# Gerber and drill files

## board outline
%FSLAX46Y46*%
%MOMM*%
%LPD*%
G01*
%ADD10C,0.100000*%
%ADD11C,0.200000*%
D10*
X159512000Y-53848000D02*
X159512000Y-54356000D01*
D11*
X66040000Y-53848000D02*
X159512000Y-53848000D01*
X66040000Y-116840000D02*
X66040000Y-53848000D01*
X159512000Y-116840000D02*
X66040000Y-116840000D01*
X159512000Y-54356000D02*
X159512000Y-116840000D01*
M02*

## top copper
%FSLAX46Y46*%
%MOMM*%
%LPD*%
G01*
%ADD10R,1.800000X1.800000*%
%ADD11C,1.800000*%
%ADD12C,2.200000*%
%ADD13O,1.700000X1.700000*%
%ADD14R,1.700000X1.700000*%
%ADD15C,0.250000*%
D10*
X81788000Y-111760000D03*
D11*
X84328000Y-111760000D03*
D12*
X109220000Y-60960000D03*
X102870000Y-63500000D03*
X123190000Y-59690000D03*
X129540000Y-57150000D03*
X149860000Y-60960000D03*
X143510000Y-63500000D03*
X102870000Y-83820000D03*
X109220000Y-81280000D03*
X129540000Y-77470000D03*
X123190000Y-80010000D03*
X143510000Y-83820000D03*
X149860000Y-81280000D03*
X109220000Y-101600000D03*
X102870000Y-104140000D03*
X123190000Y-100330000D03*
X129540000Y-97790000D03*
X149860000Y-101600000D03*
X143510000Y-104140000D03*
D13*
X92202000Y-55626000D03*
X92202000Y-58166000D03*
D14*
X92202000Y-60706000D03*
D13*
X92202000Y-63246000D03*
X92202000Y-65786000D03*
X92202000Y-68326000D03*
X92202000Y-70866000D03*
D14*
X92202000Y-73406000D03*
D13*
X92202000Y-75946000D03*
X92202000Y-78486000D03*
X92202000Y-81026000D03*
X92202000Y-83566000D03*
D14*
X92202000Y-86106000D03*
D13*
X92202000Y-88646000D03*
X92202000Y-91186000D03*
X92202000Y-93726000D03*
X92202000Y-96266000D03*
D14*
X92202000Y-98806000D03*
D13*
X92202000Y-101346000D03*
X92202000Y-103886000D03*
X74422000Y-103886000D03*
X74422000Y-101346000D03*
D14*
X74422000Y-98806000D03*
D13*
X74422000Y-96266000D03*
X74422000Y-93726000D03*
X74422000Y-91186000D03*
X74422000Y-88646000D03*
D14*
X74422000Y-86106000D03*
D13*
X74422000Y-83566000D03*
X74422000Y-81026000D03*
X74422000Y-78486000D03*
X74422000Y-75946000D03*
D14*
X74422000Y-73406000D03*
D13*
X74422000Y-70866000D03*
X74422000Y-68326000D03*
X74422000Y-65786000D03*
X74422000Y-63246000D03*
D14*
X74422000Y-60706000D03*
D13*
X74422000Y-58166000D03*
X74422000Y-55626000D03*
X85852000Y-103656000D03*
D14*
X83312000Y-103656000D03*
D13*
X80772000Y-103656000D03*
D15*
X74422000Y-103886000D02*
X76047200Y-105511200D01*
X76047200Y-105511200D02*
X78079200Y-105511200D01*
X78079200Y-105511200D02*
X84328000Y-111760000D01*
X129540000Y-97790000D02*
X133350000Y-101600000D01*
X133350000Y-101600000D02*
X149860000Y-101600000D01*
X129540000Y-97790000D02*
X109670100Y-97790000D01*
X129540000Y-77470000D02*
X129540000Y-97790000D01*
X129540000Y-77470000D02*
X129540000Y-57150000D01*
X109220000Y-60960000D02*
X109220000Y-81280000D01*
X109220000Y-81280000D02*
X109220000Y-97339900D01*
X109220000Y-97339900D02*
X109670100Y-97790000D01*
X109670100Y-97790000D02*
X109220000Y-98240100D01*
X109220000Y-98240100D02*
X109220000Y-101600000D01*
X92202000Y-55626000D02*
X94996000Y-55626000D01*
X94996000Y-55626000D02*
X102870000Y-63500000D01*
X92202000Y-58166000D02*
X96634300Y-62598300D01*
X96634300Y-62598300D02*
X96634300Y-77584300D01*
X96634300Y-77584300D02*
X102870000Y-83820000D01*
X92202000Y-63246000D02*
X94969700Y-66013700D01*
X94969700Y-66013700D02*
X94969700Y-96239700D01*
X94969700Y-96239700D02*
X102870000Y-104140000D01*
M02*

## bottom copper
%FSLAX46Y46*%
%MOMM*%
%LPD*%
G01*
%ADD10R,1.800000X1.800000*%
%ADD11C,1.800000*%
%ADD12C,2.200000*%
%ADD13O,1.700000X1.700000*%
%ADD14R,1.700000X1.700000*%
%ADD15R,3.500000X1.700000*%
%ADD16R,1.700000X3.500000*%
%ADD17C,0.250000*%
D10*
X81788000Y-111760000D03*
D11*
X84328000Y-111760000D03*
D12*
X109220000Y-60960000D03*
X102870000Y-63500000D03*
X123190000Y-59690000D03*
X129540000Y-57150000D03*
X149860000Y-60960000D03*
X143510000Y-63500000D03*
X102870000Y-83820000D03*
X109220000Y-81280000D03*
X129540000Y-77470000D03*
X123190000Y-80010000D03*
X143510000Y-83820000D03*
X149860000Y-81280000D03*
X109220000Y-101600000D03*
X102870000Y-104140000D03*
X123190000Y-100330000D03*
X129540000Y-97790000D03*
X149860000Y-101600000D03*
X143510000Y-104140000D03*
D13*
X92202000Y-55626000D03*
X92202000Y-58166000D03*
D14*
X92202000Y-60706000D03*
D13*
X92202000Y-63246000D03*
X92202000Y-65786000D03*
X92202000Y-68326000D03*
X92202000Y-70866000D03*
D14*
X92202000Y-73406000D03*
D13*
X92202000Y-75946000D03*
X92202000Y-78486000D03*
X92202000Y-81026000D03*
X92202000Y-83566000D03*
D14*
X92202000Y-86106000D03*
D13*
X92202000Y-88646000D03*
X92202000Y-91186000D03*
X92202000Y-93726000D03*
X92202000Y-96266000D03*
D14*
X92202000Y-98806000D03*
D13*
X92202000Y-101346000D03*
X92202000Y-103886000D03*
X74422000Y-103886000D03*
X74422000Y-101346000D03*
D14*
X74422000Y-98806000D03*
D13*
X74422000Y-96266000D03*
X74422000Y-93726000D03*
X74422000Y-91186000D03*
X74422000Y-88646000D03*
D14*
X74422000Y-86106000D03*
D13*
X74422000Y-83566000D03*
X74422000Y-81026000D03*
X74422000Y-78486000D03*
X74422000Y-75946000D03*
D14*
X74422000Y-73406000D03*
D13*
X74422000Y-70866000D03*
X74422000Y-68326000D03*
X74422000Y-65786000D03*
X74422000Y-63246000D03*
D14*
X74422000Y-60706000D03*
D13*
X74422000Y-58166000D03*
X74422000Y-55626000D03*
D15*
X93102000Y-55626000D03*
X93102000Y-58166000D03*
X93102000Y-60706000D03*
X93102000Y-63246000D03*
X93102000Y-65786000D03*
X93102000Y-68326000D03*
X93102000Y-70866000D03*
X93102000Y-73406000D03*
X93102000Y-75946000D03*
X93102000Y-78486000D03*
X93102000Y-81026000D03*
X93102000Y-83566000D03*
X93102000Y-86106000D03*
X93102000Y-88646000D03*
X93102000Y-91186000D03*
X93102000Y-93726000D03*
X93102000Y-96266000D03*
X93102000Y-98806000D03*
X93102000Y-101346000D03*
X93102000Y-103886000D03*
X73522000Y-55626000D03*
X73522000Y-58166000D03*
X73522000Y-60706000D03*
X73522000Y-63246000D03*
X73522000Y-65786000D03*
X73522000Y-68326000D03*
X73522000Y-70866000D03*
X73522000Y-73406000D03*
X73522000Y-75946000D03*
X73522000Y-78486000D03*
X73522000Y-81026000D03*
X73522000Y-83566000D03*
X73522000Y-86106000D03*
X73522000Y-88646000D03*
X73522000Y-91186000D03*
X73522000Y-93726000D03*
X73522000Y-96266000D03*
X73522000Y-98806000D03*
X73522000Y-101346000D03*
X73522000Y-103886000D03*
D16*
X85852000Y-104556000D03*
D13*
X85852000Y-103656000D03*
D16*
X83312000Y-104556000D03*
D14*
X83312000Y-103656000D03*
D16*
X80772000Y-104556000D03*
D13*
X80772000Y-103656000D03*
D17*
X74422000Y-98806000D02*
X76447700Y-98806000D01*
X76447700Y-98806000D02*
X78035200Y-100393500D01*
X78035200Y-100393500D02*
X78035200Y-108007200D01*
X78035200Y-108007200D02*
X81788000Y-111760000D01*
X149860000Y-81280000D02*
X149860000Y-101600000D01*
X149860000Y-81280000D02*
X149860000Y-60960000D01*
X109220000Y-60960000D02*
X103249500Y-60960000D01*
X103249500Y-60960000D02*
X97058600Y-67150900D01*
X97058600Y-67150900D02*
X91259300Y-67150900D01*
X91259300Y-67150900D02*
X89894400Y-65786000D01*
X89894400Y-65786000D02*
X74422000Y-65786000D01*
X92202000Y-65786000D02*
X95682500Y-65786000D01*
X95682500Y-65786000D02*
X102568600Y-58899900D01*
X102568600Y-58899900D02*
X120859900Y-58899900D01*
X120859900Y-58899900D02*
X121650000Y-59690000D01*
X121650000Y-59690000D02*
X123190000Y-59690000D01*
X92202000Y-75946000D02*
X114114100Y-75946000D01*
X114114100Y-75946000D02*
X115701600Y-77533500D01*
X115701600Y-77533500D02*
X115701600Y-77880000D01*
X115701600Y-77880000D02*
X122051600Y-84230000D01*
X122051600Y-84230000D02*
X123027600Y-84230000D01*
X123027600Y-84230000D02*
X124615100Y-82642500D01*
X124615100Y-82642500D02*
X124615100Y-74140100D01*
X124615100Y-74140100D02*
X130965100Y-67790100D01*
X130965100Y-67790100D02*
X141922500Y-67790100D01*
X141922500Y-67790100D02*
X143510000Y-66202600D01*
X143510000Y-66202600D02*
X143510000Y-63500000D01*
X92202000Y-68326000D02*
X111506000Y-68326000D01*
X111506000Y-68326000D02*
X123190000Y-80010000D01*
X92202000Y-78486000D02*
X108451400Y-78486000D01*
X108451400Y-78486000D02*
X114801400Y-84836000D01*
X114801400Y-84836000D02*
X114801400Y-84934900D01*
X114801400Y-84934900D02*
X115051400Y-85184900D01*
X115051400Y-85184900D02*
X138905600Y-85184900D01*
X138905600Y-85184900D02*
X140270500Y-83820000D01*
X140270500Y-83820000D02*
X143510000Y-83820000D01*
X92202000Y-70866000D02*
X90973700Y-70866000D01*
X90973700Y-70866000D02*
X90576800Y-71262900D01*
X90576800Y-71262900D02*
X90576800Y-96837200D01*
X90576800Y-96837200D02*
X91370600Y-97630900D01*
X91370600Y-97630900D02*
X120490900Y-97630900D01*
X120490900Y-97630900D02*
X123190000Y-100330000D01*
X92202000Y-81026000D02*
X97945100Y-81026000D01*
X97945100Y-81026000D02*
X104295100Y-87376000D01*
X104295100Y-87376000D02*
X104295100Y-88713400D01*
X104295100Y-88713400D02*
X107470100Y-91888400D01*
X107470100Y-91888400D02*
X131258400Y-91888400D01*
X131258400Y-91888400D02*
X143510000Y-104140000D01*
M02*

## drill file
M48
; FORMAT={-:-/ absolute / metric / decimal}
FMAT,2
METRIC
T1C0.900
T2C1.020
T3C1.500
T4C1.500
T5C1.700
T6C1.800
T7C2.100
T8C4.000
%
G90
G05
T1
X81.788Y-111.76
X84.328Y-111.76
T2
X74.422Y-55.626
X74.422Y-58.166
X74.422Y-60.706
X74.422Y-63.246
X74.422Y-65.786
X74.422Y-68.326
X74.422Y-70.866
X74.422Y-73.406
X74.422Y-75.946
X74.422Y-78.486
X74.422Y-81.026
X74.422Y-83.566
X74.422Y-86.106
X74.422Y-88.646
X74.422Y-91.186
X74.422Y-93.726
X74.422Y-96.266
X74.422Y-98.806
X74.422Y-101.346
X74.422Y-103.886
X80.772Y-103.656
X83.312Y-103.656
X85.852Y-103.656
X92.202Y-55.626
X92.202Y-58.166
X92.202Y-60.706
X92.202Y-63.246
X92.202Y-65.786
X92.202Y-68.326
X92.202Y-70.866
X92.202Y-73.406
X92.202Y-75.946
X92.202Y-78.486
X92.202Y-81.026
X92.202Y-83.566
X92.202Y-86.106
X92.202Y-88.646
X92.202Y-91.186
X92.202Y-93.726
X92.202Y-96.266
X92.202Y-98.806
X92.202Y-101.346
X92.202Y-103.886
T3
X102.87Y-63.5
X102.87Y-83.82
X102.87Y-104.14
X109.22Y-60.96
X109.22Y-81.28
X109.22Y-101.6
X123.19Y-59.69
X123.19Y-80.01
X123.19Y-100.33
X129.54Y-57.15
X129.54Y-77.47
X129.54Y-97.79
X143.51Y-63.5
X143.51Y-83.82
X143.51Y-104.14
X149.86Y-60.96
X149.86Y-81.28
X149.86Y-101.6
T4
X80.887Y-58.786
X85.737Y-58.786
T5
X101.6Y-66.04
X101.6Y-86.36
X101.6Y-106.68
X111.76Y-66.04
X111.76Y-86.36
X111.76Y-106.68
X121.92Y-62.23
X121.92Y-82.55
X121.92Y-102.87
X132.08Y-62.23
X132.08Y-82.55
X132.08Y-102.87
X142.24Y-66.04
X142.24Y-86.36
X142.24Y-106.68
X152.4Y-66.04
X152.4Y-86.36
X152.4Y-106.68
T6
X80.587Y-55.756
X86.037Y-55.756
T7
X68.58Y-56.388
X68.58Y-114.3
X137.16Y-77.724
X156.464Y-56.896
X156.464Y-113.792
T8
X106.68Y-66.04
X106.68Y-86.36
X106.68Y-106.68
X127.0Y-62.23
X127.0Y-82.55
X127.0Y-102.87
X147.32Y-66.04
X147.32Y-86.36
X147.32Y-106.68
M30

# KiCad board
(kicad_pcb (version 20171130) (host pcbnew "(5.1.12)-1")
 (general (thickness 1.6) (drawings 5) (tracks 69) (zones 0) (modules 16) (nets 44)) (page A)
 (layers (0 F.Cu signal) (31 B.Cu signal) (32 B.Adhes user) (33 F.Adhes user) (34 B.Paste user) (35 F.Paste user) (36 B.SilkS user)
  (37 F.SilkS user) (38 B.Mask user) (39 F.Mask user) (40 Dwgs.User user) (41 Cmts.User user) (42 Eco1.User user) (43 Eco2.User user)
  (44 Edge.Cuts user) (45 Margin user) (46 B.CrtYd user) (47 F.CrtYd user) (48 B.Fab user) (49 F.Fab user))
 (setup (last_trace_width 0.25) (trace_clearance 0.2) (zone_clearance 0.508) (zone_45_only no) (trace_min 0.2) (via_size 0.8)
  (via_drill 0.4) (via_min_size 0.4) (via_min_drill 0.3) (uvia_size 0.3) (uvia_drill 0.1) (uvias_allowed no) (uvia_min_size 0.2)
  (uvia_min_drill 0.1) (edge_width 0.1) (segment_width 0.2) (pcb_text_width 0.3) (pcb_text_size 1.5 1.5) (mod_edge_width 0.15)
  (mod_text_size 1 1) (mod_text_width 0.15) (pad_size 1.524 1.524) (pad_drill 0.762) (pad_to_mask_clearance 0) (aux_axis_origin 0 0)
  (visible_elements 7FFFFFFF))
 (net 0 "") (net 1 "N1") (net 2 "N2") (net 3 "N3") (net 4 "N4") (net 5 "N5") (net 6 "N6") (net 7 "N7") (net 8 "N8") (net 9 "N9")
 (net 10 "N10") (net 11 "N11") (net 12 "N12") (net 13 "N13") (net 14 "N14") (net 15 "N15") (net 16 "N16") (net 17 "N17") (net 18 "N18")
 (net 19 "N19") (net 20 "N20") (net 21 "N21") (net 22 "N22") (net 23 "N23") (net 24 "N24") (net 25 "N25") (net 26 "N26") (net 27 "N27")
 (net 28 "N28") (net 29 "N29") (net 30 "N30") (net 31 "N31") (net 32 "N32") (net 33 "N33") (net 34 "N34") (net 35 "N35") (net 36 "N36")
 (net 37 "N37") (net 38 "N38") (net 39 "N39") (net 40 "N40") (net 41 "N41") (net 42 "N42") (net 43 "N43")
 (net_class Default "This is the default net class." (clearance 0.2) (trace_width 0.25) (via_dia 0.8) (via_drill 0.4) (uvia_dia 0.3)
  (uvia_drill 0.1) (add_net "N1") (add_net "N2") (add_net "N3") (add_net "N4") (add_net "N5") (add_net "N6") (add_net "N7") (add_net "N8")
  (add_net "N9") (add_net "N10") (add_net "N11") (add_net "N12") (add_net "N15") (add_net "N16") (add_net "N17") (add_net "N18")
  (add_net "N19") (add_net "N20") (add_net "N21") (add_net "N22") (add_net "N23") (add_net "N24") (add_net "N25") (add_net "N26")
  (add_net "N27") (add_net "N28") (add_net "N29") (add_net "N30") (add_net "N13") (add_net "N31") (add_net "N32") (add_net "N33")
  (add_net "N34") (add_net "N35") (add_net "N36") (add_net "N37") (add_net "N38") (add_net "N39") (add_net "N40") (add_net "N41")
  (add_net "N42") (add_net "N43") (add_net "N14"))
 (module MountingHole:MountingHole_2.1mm (layer F.Cu) (at 137.16 77.724)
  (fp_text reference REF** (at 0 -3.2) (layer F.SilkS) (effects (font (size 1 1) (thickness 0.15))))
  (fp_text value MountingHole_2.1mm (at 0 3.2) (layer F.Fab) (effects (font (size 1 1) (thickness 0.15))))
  (pad "" np_thru_hole circle (at 0 0) (size 2.1 2.1) (drill 2.1) (layers *.Cu *.Mask)))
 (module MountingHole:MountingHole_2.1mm (layer F.Cu) (at 68.58 56.388)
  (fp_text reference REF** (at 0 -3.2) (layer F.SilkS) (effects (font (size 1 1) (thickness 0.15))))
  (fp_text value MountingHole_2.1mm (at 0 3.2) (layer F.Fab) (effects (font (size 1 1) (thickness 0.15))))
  (pad "" np_thru_hole circle (at 0 0) (size 2.1 2.1) (drill 2.1) (layers *.Cu *.Mask)))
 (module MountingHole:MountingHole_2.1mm (layer F.Cu) (at 156.464 113.792)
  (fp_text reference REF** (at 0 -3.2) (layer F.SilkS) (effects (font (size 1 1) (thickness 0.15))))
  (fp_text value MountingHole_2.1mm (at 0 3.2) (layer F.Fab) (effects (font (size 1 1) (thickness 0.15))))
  (pad "" np_thru_hole circle (at 0 0) (size 2.1 2.1) (drill 2.1) (layers *.Cu *.Mask)))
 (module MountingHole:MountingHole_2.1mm (layer F.Cu) (at 156.464 56.896)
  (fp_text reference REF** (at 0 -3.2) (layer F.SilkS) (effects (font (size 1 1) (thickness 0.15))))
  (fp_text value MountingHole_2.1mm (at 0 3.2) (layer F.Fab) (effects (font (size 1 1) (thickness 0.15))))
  (pad "" np_thru_hole circle (at 0 0) (size 2.1 2.1) (drill 2.1) (layers *.Cu *.Mask)))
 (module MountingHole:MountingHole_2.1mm (layer F.Cu) (at 68.58 114.3)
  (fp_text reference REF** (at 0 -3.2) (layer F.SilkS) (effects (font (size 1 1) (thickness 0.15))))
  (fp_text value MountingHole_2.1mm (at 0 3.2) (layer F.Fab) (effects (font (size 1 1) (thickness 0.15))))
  (pad "" np_thru_hole circle (at 0 0) (size 2.1 2.1) (drill 2.1) (layers *.Cu *.Mask)))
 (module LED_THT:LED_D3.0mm (layer F.Cu) (at 81.788 111.76)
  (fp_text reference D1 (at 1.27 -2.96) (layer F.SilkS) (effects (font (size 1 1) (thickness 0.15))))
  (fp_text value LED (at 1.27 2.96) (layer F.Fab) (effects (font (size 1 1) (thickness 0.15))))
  (pad 1 thru_hole rect (at 0 0) (size 1.8 1.8) (drill 0.9) (layers *.Cu *.Mask) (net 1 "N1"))
  (pad 2 thru_hole circle (at 2.54 0) (size 1.8 1.8) (drill 0.9) (layers *.Cu *.Mask) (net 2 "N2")))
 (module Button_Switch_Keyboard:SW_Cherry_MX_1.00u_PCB (layer F.Cu) (at 109.22 60.96)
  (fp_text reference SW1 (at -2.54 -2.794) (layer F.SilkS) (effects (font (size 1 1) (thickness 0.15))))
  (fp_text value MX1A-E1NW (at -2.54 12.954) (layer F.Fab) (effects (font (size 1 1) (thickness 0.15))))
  (pad 1 thru_hole circle (at 0 0) (size 2.2 2.2) (drill 1.5) (layers *.Cu *.Mask) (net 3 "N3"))
  (pad 2 thru_hole circle (at -6.35 2.54) (size 2.2 2.2) (drill 1.5) (layers *.Cu *.Mask) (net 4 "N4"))
  (pad "" np_thru_hole circle (at -2.54 5.08) (size 4 4) (drill 4) (layers *.Cu *.Mask))
  (pad "" np_thru_hole circle (at -7.62 5.08) (size 1.7 1.7) (drill 1.7) (layers *.Cu *.Mask))
  (pad "" np_thru_hole circle (at 2.54 5.08) (size 1.7 1.7) (drill 1.7) (layers *.Cu *.Mask)))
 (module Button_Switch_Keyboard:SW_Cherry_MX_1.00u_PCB (layer F.Cu) (at 129.54 57.15)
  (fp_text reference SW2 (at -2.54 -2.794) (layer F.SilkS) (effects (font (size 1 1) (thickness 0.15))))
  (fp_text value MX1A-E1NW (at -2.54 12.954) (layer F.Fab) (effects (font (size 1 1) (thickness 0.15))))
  (pad "" np_thru_hole circle (at 2.54 5.08) (size 1.7 1.7) (drill 1.7) (layers *.Cu *.Mask))
  (pad "" np_thru_hole circle (at -7.62 5.08) (size 1.7 1.7) (drill 1.7) (layers *.Cu *.Mask))
  (pad "" np_thru_hole circle (at -2.54 5.08) (size 4 4) (drill 4) (layers *.Cu *.Mask))
  (pad 2 thru_hole circle (at -6.35 2.54) (size 2.2 2.2) (drill 1.5) (layers *.Cu *.Mask) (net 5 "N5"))
  (pad 1 thru_hole circle (at 0 0) (size 2.2 2.2) (drill 1.5) (layers *.Cu *.Mask) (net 3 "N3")))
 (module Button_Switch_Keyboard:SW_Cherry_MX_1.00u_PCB (layer F.Cu) (at 149.86 60.96)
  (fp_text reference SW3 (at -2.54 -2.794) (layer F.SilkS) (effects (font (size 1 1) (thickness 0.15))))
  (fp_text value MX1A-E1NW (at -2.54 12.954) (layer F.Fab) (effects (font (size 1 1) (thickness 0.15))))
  (pad 1 thru_hole circle (at 0 0) (size 2.2 2.2) (drill 1.5) (layers *.Cu *.Mask) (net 3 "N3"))
  (pad 2 thru_hole circle (at -6.35 2.54) (size 2.2 2.2) (drill 1.5) (layers *.Cu *.Mask) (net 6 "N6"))
  (pad "" np_thru_hole circle (at -2.54 5.08) (size 4 4) (drill 4) (layers *.Cu *.Mask))
  (pad "" np_thru_hole circle (at -7.62 5.08) (size 1.7 1.7) (drill 1.7) (layers *.Cu *.Mask))
  (pad "" np_thru_hole circle (at 2.54 5.08) (size 1.7 1.7) (drill 1.7) (layers *.Cu *.Mask)))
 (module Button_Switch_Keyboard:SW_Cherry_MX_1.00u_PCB (layer F.Cu) (at 109.22 81.28)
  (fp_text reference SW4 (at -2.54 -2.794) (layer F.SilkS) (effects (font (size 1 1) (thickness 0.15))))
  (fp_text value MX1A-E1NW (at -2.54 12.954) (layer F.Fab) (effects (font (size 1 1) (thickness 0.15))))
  (pad "" np_thru_hole circle (at 2.54 5.08) (size 1.7 1.7) (drill 1.7) (layers *.Cu *.Mask))
  (pad "" np_thru_hole circle (at -7.62 5.08) (size 1.7 1.7) (drill 1.7) (layers *.Cu *.Mask))
  (pad "" np_thru_hole circle (at -2.54 5.08) (size 4 4) (drill 4) (layers *.Cu *.Mask))
  (pad 2 thru_hole circle (at -6.35 2.54) (size 2.2 2.2) (drill 1.5) (layers *.Cu *.Mask) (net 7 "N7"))
  (pad 1 thru_hole circle (at 0 0) (size 2.2 2.2) (drill 1.5) (layers *.Cu *.Mask) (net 3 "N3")))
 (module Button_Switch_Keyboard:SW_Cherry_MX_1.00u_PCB (layer F.Cu) (at 129.54 77.47)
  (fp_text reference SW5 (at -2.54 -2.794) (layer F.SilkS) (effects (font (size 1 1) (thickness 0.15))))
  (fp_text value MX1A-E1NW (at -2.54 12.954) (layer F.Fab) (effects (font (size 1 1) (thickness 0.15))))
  (pad 1 thru_hole circle (at 0 0) (size 2.2 2.2) (drill 1.5) (layers *.Cu *.Mask) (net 3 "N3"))
  (pad 2 thru_hole circle (at -6.35 2.54) (size 2.2 2.2) (drill 1.5) (layers *.Cu *.Mask) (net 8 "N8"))
  (pad "" np_thru_hole circle (at -2.54 5.08) (size 4 4) (drill 4) (layers *.Cu *.Mask))
  (pad "" np_thru_hole circle (at -7.62 5.08) (size 1.7 1.7) (drill 1.7) (layers *.Cu *.Mask))
  (pad "" np_thru_hole circle (at 2.54 5.08) (size 1.7 1.7) (drill 1.7) (layers *.Cu *.Mask)))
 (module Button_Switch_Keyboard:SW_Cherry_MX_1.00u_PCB (layer F.Cu) (at 149.86 81.28)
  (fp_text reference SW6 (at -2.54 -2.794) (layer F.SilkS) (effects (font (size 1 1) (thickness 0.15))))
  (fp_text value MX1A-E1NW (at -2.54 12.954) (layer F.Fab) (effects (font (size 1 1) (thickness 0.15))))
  (pad "" np_thru_hole circle (at 2.54 5.08) (size 1.7 1.7) (drill 1.7) (layers *.Cu *.Mask))
  (pad "" np_thru_hole circle (at -7.62 5.08) (size 1.7 1.7) (drill 1.7) (layers *.Cu *.Mask))
  (pad "" np_thru_hole circle (at -2.54 5.08) (size 4 4) (drill 4) (layers *.Cu *.Mask))
  (pad 2 thru_hole circle (at -6.35 2.54) (size 2.2 2.2) (drill 1.5) (layers *.Cu *.Mask) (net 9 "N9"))
  (pad 1 thru_hole circle (at 0 0) (size 2.2 2.2) (drill 1.5) (layers *.Cu *.Mask) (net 3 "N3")))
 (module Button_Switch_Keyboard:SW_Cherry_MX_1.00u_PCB (layer F.Cu) (at 109.22 101.6)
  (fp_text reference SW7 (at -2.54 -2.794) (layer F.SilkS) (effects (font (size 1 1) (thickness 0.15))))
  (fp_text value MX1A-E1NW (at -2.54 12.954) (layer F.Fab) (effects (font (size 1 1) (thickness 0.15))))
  (pad 1 thru_hole circle (at 0 0) (size 2.2 2.2) (drill 1.5) (layers *.Cu *.Mask) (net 3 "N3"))
  (pad 2 thru_hole circle (at -6.35 2.54) (size 2.2 2.2) (drill 1.5) (layers *.Cu *.Mask) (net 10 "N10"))
  (pad "" np_thru_hole circle (at -2.54 5.08) (size 4 4) (drill 4) (layers *.Cu *.Mask))
  (pad "" np_thru_hole circle (at -7.62 5.08) (size 1.7 1.7) (drill 1.7) (layers *.Cu *.Mask))
  (pad "" np_thru_hole circle (at 2.54 5.08) (size 1.7 1.7) (drill 1.7) (layers *.Cu *.Mask)))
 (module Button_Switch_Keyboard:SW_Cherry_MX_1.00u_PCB (layer F.Cu) (at 129.54 97.79)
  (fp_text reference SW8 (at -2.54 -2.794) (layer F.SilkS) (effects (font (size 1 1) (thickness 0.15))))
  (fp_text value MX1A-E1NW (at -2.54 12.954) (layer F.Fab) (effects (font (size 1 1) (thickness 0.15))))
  (pad "" np_thru_hole circle (at 2.54 5.08) (size 1.7 1.7) (drill 1.7) (layers *.Cu *.Mask))
  (pad "" np_thru_hole circle (at -7.62 5.08) (size 1.7 1.7) (drill 1.7) (layers *.Cu *.Mask))
  (pad "" np_thru_hole circle (at -2.54 5.08) (size 4 4) (drill 4) (layers *.Cu *.Mask))
  (pad 2 thru_hole circle (at -6.35 2.54) (size 2.2 2.2) (drill 1.5) (layers *.Cu *.Mask) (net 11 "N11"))
  (pad 1 thru_hole circle (at 0 0) (size 2.2 2.2) (drill 1.5) (layers *.Cu *.Mask) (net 3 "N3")))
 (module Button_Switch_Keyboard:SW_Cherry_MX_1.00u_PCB (layer F.Cu) (at 149.86 101.6)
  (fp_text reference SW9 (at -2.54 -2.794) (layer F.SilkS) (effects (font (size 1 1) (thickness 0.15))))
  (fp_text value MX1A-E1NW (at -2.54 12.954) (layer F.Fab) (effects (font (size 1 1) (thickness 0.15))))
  (pad 1 thru_hole circle (at 0 0) (size 2.2 2.2) (drill 1.5) (layers *.Cu *.Mask) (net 3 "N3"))
  (pad 2 thru_hole circle (at -6.35 2.54) (size 2.2 2.2) (drill 1.5) (layers *.Cu *.Mask) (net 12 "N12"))
  (pad "" np_thru_hole circle (at -2.54 5.08) (size 4 4) (drill 4) (layers *.Cu *.Mask))
  (pad "" np_thru_hole circle (at -7.62 5.08) (size 1.7 1.7) (drill 1.7) (layers *.Cu *.Mask))
  (pad "" np_thru_hole circle (at 2.54 5.08) (size 1.7 1.7) (drill 1.7) (layers *.Cu *.Mask)))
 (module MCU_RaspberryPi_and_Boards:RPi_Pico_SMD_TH (layer B.Cu) (at 83.312 79.756 180)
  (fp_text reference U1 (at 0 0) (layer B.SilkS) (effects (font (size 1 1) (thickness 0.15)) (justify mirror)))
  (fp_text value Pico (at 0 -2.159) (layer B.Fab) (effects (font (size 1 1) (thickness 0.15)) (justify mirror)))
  (pad 1 thru_hole oval (at -8.89 24.13 180) (size 1.7 1.7) (drill 1.02) (layers *.Cu *.Mask) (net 4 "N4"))
  (pad 2 thru_hole oval (at -8.89 21.59 180) (size 1.7 1.7) (drill 1.02) (layers *.Cu *.Mask) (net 7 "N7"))
  (pad 3 thru_hole rect (at -8.89 19.05 180) (size 1.7 1.7) (drill 1.02) (layers *.Cu *.Mask) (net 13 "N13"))
  (pad 4 thru_hole oval (at -8.89 16.51 180) (size 1.7 1.7) (drill 1.02) (layers *.Cu *.Mask) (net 10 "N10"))
  (pad 5 thru_hole oval (at -8.89 13.97 180) (size 1.7 1.7) (drill 1.02) (layers *.Cu *.Mask) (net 5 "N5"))
  (pad 6 thru_hole oval (at -8.89 11.43 180) (size 1.7 1.7) (drill 1.02) (layers *.Cu *.Mask) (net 8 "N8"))
  (pad 7 thru_hole oval (at -8.89 8.89 180) (size 1.7 1.7) (drill 1.02) (layers *.Cu *.Mask) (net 11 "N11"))
  (pad 8 thru_hole rect (at -8.89 6.35 180) (size 1.7 1.7) (drill 1.02) (layers *.Cu *.Mask) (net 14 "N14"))
  (pad 9 thru_hole oval (at -8.89 3.81 180) (size 1.7 1.7) (drill 1.02) (layers *.Cu *.Mask) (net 6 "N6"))
  (pad 10 thru_hole oval (at -8.89 1.27 180) (size 1.7 1.7) (drill 1.02) (layers *.Cu *.Mask) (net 9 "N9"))
  (pad 11 thru_hole oval (at -8.89 -1.27 180) (size 1.7 1.7) (drill 1.02) (layers *.Cu *.Mask) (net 12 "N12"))
  (pad 12 thru_hole oval (at -8.89 -3.81 180) (size 1.7 1.7) (drill 1.02) (layers *.Cu *.Mask) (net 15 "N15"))
  (pad 13 thru_hole rect (at -8.89 -6.35 180) (size 1.7 1.7) (drill 1.02) (layers *.Cu *.Mask) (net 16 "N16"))
  (pad 14 thru_hole oval (at -8.89 -8.89 180) (size 1.7 1.7) (drill 1.02) (layers *.Cu *.Mask) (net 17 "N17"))
  (pad 15 thru_hole oval (at -8.89 -11.43 180) (size 1.7 1.7) (drill 1.02) (layers *.Cu *.Mask) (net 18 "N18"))
  (pad 16 thru_hole oval (at -8.89 -13.97 180) (size 1.7 1.7) (drill 1.02) (layers *.Cu *.Mask) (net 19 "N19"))
  (pad 17 thru_hole oval (at -8.89 -16.51 180) (size 1.7 1.7) (drill 1.02) (layers *.Cu *.Mask) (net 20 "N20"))
  (pad 18 thru_hole rect (at -8.89 -19.05 180) (size 1.7 1.7) (drill 1.02) (layers *.Cu *.Mask) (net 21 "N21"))
  (pad 19 thru_hole oval (at -8.89 -21.59 180) (size 1.7 1.7) (drill 1.02) (layers *.Cu *.Mask) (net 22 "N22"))
  (pad 20 thru_hole oval (at -8.89 -24.13 180) (size 1.7 1.7) (drill 1.02) (layers *.Cu *.Mask) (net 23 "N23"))
  (pad 21 thru_hole oval (at 8.89 -24.13 180) (size 1.7 1.7) (drill 1.02) (layers *.Cu *.Mask) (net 2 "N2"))
  (pad 22 thru_hole oval (at 8.89 -21.59 180) (size 1.7 1.7) (drill 1.02) (layers *.Cu *.Mask) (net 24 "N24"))
  (pad 23 thru_hole rect (at 8.89 -19.05 180) (size 1.7 1.7) (drill 1.02) (layers *.Cu *.Mask) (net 1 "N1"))
  (pad 24 thru_hole oval (at 8.89 -16.51 180) (size 1.7 1.7) (drill 1.02) (layers *.Cu *.Mask) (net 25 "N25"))
  (pad 25 thru_hole oval (at 8.89 -13.97 180) (size 1.7 1.7) (drill 1.02) (layers *.Cu *.Mask) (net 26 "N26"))
  (pad 26 thru_hole oval (at 8.89 -11.43 180) (size 1.7 1.7) (drill 1.02) (layers *.Cu *.Mask) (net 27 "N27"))
  (pad 27 thru_hole oval (at 8.89 -8.89 180) (size 1.7 1.7) (drill 1.02) (layers *.Cu *.Mask) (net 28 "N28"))
  (pad 28 thru_hole rect (at 8.89 -6.35 180) (size 1.7 1.7) (drill 1.02) (layers *.Cu *.Mask) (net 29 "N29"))
  (pad 29 thru_hole oval (at 8.89 -3.81 180) (size 1.7 1.7) (drill 1.02) (layers *.Cu *.Mask) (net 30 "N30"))
  (pad 30 thru_hole oval (at 8.89 -1.27 180) (size 1.7 1.7) (drill 1.02) (layers *.Cu *.Mask) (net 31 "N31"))
  (pad 31 thru_hole oval (at 8.89 1.27 180) (size 1.7 1.7) (drill 1.02) (layers *.Cu *.Mask) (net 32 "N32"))
  (pad 32 thru_hole oval (at 8.89 3.81 180) (size 1.7 1.7) (drill 1.02) (layers *.Cu *.Mask) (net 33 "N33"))
  (pad 33 thru_hole rect (at 8.89 6.35 180) (size 1.7 1.7) (drill 1.02) (layers *.Cu *.Mask) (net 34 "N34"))
  (pad 34 thru_hole oval (at 8.89 8.89 180) (size 1.7 1.7) (drill 1.02) (layers *.Cu *.Mask) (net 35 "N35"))
  (pad 35 thru_hole oval (at 8.89 11.43 180) (size 1.7 1.7) (drill 1.02) (layers *.Cu *.Mask) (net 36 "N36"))
  (pad 36 thru_hole oval (at 8.89 13.97 180) (size 1.7 1.7) (drill 1.02) (layers *.Cu *.Mask) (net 3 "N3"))
  (pad 37 thru_hole oval (at 8.89 16.51 180) (size 1.7 1.7) (drill 1.02) (layers *.Cu *.Mask) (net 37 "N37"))
  (pad 38 thru_hole rect (at 8.89 19.05 180) (size 1.7 1.7) (drill 1.02) (layers *.Cu *.Mask) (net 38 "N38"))
  (pad 39 thru_hole oval (at 8.89 21.59 180) (size 1.7 1.7) (drill 1.02) (layers *.Cu *.Mask) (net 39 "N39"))
  (pad 40 thru_hole oval (at 8.89 24.13 180) (size 1.7 1.7) (drill 1.02) (layers *.Cu *.Mask) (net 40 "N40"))
  (pad 1 smd rect (at -8.89 24.13 180) (size 3.5 1.7) (drill (offset -0.9 0)) (layers B.Cu B.Mask) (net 4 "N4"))
  (pad 2 smd rect (at -8.89 21.59 180) (size 3.5 1.7) (drill (offset -0.9 0)) (layers B.Cu B.Mask) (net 7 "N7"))
  (pad 3 smd rect (at -8.89 19.05 180) (size 3.5 1.7) (drill (offset -0.9 0)) (layers B.Cu B.Mask) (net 13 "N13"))
  (pad 4 smd rect (at -8.89 16.51 180) (size 3.5 1.7) (drill (offset -0.9 0)) (layers B.Cu B.Mask) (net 10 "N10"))
  (pad 5 smd rect (at -8.89 13.97 180) (size 3.5 1.7) (drill (offset -0.9 0)) (layers B.Cu B.Mask) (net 5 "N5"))
  (pad 6 smd rect (at -8.89 11.43 180) (size 3.5 1.7) (drill (offset -0.9 0)) (layers B.Cu B.Mask) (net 8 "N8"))
  (pad 7 smd rect (at -8.89 8.89 180) (size 3.5 1.7) (drill (offset -0.9 0)) (layers B.Cu B.Mask) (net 11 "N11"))
  (pad 8 smd rect (at -8.89 6.35 180) (size 3.5 1.7) (drill (offset -0.9 0)) (layers B.Cu B.Mask) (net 14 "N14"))
  (pad 9 smd rect (at -8.89 3.81 180) (size 3.5 1.7) (drill (offset -0.9 0)) (layers B.Cu B.Mask) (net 6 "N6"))
  (pad 10 smd rect (at -8.89 1.27 180) (size 3.5 1.7) (drill (offset -0.9 0)) (layers B.Cu B.Mask) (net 9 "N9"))
  (pad 11 smd rect (at -8.89 -1.27 180) (size 3.5 1.7) (drill (offset -0.9 0)) (layers B.Cu B.Mask) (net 12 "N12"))
  (pad 12 smd rect (at -8.89 -3.81 180) (size 3.5 1.7) (drill (offset -0.9 0)) (layers B.Cu B.Mask) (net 15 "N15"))
  (pad 13 smd rect (at -8.89 -6.35 180) (size 3.5 1.7) (drill (offset -0.9 0)) (layers B.Cu B.Mask) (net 16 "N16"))
  (pad 14 smd rect (at -8.89 -8.89 180) (size 3.5 1.7) (drill (offset -0.9 0)) (layers B.Cu B.Mask) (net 17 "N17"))
  (pad 15 smd rect (at -8.89 -11.43 180) (size 3.5 1.7) (drill (offset -0.9 0)) (layers B.Cu B.Mask) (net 18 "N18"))
  (pad 16 smd rect (at -8.89 -13.97 180) (size 3.5 1.7) (drill (offset -0.9 0)) (layers B.Cu B.Mask) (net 19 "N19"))
  (pad 17 smd rect (at -8.89 -16.51 180) (size 3.5 1.7) (drill (offset -0.9 0)) (layers B.Cu B.Mask) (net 20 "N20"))
  (pad 18 smd rect (at -8.89 -19.05 180) (size 3.5 1.7) (drill (offset -0.9 0)) (layers B.Cu B.Mask) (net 21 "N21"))
  (pad 19 smd rect (at -8.89 -21.59 180) (size 3.5 1.7) (drill (offset -0.9 0)) (layers B.Cu B.Mask) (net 22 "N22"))
  (pad 20 smd rect (at -8.89 -24.13 180) (size 3.5 1.7) (drill (offset -0.9 0)) (layers B.Cu B.Mask) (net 23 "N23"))
  (pad 40 smd rect (at 8.89 24.13 180) (size 3.5 1.7) (drill (offset 0.9 0)) (layers B.Cu B.Mask) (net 40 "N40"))
  (pad 39 smd rect (at 8.89 21.59 180) (size 3.5 1.7) (drill (offset 0.9 0)) (layers B.Cu B.Mask) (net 39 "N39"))
  (pad 38 smd rect (at 8.89 19.05 180) (size 3.5 1.7) (drill (offset 0.9 0)) (layers B.Cu B.Mask) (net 38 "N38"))
  (pad 37 smd rect (at 8.89 16.51 180) (size 3.5 1.7) (drill (offset 0.9 0)) (layers B.Cu B.Mask) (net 37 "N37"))
  (pad 36 smd rect (at 8.89 13.97 180) (size 3.5 1.7) (drill (offset 0.9 0)) (layers B.Cu B.Mask) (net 3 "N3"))
  (pad 35 smd rect (at 8.89 11.43 180) (size 3.5 1.7) (drill (offset 0.9 0)) (layers B.Cu B.Mask) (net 36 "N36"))
  (pad 34 smd rect (at 8.89 8.89 180) (size 3.5 1.7) (drill (offset 0.9 0)) (layers B.Cu B.Mask) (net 35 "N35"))
  (pad 33 smd rect (at 8.89 6.35 180) (size 3.5 1.7) (drill (offset 0.9 0)) (layers B.Cu B.Mask) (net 34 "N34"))
  (pad 32 smd rect (at 8.89 3.81 180) (size 3.5 1.7) (drill (offset 0.9 0)) (layers B.Cu B.Mask) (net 33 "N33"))
  (pad 31 smd rect (at 8.89 1.27 180) (size 3.5 1.7) (drill (offset 0.9 0)) (layers B.Cu B.Mask) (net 32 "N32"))
  (pad 30 smd rect (at 8.89 -1.27 180) (size 3.5 1.7) (drill (offset 0.9 0)) (layers B.Cu B.Mask) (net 31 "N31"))
  (pad 29 smd rect (at 8.89 -3.81 180) (size 3.5 1.7) (drill (offset 0.9 0)) (layers B.Cu B.Mask) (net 30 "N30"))
  (pad 28 smd rect (at 8.89 -6.35 180) (size 3.5 1.7) (drill (offset 0.9 0)) (layers B.Cu B.Mask) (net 29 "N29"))
  (pad 27 smd rect (at 8.89 -8.89 180) (size 3.5 1.7) (drill (offset 0.9 0)) (layers B.Cu B.Mask) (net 28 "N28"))
  (pad 26 smd rect (at 8.89 -11.43 180) (size 3.5 1.7) (drill (offset 0.9 0)) (layers B.Cu B.Mask) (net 27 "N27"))
  (pad 25 smd rect (at 8.89 -13.97 180) (size 3.5 1.7) (drill (offset 0.9 0)) (layers B.Cu B.Mask) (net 26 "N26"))
  (pad 24 smd rect (at 8.89 -16.51 180) (size 3.5 1.7) (drill (offset 0.9 0)) (layers B.Cu B.Mask) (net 25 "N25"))
  (pad 23 smd rect (at 8.89 -19.05 180) (size 3.5 1.7) (drill (offset 0.9 0)) (layers B.Cu B.Mask) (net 1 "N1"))
  (pad 22 smd rect (at 8.89 -21.59 180) (size 3.5 1.7) (drill (offset 0.9 0)) (layers B.Cu B.Mask) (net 24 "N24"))
  (pad 21 smd rect (at 8.89 -24.13 180) (size 3.5 1.7) (drill (offset 0.9 0)) (layers B.Cu B.Mask) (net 2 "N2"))
  (pad "" np_thru_hole oval (at -2.725 24 180) (size 1.8 1.8) (drill 1.8) (layers *.Cu *.Mask))
  (pad "" np_thru_hole oval (at 2.725 24 180) (size 1.8 1.8) (drill 1.8) (layers *.Cu *.Mask))
  (pad "" np_thru_hole oval (at -2.425 20.97 180) (size 1.5 1.5) (drill 1.5) (layers *.Cu *.Mask))
  (pad "" np_thru_hole oval (at 2.425 20.97 180) (size 1.5 1.5) (drill 1.5) (layers *.Cu *.Mask))
  (pad 41 smd rect (at -2.54 -23.9 90) (size 3.5 1.7) (drill (offset -0.9 0)) (layers B.Cu B.Mask) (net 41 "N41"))
  (pad 41 thru_hole oval (at -2.54 -23.9 180) (size 1.7 1.7) (drill 1.02) (layers *.Cu *.Mask) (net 41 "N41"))
  (pad 42 smd rect (at 0 -23.9 90) (size 3.5 1.7) (drill (offset -0.9 0)) (layers B.Cu B.Mask) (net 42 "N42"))
  (pad 42 thru_hole rect (at 0 -23.9 180) (size 1.7 1.7) (drill 1.02) (layers *.Cu *.Mask) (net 42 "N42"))
  (pad 43 smd rect (at 2.54 -23.9 90) (size 3.5 1.7) (drill (offset -0.9 0)) (layers B.Cu B.Mask) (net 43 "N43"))
  (pad 43 thru_hole oval (at 2.54 -23.9 180) (size 1.7 1.7) (drill 1.02) (layers *.Cu *.Mask) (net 43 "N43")))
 (gr_line (start 159.512 53.848) (end 159.512 54.356) (layer Edge.Cuts) (width 0.1))
 (gr_line (start 66.04 53.848) (end 159.512 53.848) (layer Edge.Cuts) (width 0.2))
 (gr_line (start 66.04 116.84) (end 66.04 53.848) (layer Edge.Cuts) (width 0.2))
 (gr_line (start 159.512 116.84) (end 66.04 116.84) (layer Edge.Cuts) (width 0.2))
 (gr_line (start 159.512 54.356) (end 159.512 116.84) (layer Edge.Cuts) (width 0.2))
 (segment (start 74.422 98.806) (end 76.4477 98.806) (width 0.25) (layer B.Cu) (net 1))
 (segment (start 76.4477 98.806) (end 78.0352 100.3935) (width 0.25) (layer B.Cu) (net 1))
 (segment (start 78.0352 100.3935) (end 78.0352 108.0072) (width 0.25) (layer B.Cu) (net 1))
 (segment (start 78.0352 108.0072) (end 81.788 111.76) (width 0.25) (layer B.Cu) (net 1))
 (segment (start 74.422 103.886) (end 76.0472 105.5112) (width 0.25) (layer F.Cu) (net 2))
 (segment (start 76.0472 105.5112) (end 78.0792 105.5112) (width 0.25) (layer F.Cu) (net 2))
 (segment (start 78.0792 105.5112) (end 84.328 111.76) (width 0.25) (layer F.Cu) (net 2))
 (segment (start 129.54 97.79) (end 133.35 101.6) (width 0.25) (layer F.Cu) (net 3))
 (segment (start 133.35 101.6) (end 149.86 101.6) (width 0.25) (layer F.Cu) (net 3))
 (segment (start 129.54 97.79) (end 109.6701 97.79) (width 0.25) (layer F.Cu) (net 3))
 (segment (start 129.54 77.47) (end 129.54 97.79) (width 0.25) (layer F.Cu) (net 3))
 (segment (start 129.54 77.47) (end 129.54 57.15) (width 0.25) (layer F.Cu) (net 3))
 (segment (start 149.86 81.28) (end 149.86 101.6) (width 0.25) (layer B.Cu) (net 3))
 (segment (start 149.86 81.28) (end 149.86 60.96) (width 0.25) (layer B.Cu) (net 3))
 (segment (start 109.22 60.96) (end 109.22 81.28) (width 0.25) (layer F.Cu) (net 3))
 (segment (start 109.22 81.28) (end 109.22 97.3399) (width 0.25) (layer F.Cu) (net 3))
 (segment (start 109.22 97.3399) (end 109.6701 97.79) (width 0.25) (layer F.Cu) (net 3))
 (segment (start 109.6701 97.79) (end 109.22 98.2401) (width 0.25) (layer F.Cu) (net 3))
 (segment (start 109.22 98.2401) (end 109.22 101.6) (width 0.25) (layer F.Cu) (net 3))
 (segment (start 109.22 60.96) (end 103.2495 60.96) (width 0.25) (layer B.Cu) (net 3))
 (segment (start 103.2495 60.96) (end 97.0586 67.1509) (width 0.25) (layer B.Cu) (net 3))
 (segment (start 97.0586 67.1509) (end 91.2593 67.1509) (width 0.25) (layer B.Cu) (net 3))
 (segment (start 91.2593 67.1509) (end 89.8944 65.786) (width 0.25) (layer B.Cu) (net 3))
 (segment (start 89.8944 65.786) (end 74.422 65.786) (width 0.25) (layer B.Cu) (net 3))
 (segment (start 92.202 55.626) (end 94.996 55.626) (width 0.25) (layer F.Cu) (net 4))
 (segment (start 94.996 55.626) (end 102.87 63.5) (width 0.25) (layer F.Cu) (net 4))
 (segment (start 92.202 65.786) (end 95.6825 65.786) (width 0.25) (layer B.Cu) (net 5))
 (segment (start 95.6825 65.786) (end 102.5686 58.8999) (width 0.25) (layer B.Cu) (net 5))
 (segment (start 102.5686 58.8999) (end 120.8599 58.8999) (width 0.25) (layer B.Cu) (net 5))
 (segment (start 120.8599 58.8999) (end 121.65 59.69) (width 0.25) (layer B.Cu) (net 5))
 (segment (start 121.65 59.69) (end 123.19 59.69) (width 0.25) (layer B.Cu) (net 5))
 (segment (start 92.202 75.946) (end 114.1141 75.946) (width 0.25) (layer B.Cu) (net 6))
 (segment (start 114.1141 75.946) (end 115.7016 77.5335) (width 0.25) (layer B.Cu) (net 6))
 (segment (start 115.7016 77.5335) (end 115.7016 77.88) (width 0.25) (layer B.Cu) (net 6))
 (segment (start 115.7016 77.88) (end 122.0516 84.23) (width 0.25) (layer B.Cu) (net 6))
 (segment (start 122.0516 84.23) (end 123.0276 84.23) (width 0.25) (layer B.Cu) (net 6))
 (segment (start 123.0276 84.23) (end 124.6151 82.6425) (width 0.25) (layer B.Cu) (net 6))
 (segment (start 124.6151 82.6425) (end 124.6151 74.1401) (width 0.25) (layer B.Cu) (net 6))
 (segment (start 124.6151 74.1401) (end 130.9651 67.7901) (width 0.25) (layer B.Cu) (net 6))
 (segment (start 130.9651 67.7901) (end 141.9225 67.7901) (width 0.25) (layer B.Cu) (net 6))
 (segment (start 141.9225 67.7901) (end 143.51 66.2026) (width 0.25) (layer B.Cu) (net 6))
 (segment (start 143.51 66.2026) (end 143.51 63.5) (width 0.25) (layer B.Cu) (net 6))
 (segment (start 92.202 58.166) (end 96.6343 62.5983) (width 0.25) (layer F.Cu) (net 7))
 (segment (start 96.6343 62.5983) (end 96.6343 77.5843) (width 0.25) (layer F.Cu) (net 7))
 (segment (start 96.6343 77.5843) (end 102.87 83.82) (width 0.25) (layer F.Cu) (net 7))
 (segment (start 92.202 68.326) (end 111.506 68.326) (width 0.25) (layer B.Cu) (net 8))
 (segment (start 111.506 68.326) (end 123.19 80.01) (width 0.25) (layer B.Cu) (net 8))
 (segment (start 92.202 78.486) (end 108.4514 78.486) (width 0.25) (layer B.Cu) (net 9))
 (segment (start 108.4514 78.486) (end 114.8014 84.836) (width 0.25) (layer B.Cu) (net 9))
 (segment (start 114.8014 84.836) (end 114.8014 84.9349) (width 0.25) (layer B.Cu) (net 9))
 (segment (start 114.8014 84.9349) (end 115.0514 85.1849) (width 0.25) (layer B.Cu) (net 9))
 (segment (start 115.0514 85.1849) (end 138.9056 85.1849) (width 0.25) (layer B.Cu) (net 9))
 (segment (start 138.9056 85.1849) (end 140.2705 83.82) (width 0.25) (layer B.Cu) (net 9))
 (segment (start 140.2705 83.82) (end 143.51 83.82) (width 0.25) (layer B.Cu) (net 9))
 (segment (start 92.202 63.246) (end 94.9697 66.0137) (width 0.25) (layer F.Cu) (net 10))
 (segment (start 94.9697 66.0137) (end 94.9697 96.2397) (width 0.25) (layer F.Cu) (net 10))
 (segment (start 94.9697 96.2397) (end 102.87 104.14) (width 0.25) (layer F.Cu) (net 10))
 (segment (start 92.202 70.866) (end 90.9737 70.866) (width 0.25) (layer B.Cu) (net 11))
 (segment (start 90.9737 70.866) (end 90.5768 71.2629) (width 0.25) (layer B.Cu) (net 11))
 (segment (start 90.5768 71.2629) (end 90.5768 96.8372) (width 0.25) (layer B.Cu) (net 11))
 (segment (start 90.5768 96.8372) (end 91.3706 97.6309) (width 0.25) (layer B.Cu) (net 11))
 (segment (start 91.3706 97.6309) (end 120.4909 97.6309) (width 0.25) (layer B.Cu) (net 11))
 (segment (start 120.4909 97.6309) (end 123.19 100.33) (width 0.25) (layer B.Cu) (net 11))
 (segment (start 92.202 81.026) (end 97.9451 81.026) (width 0.25) (layer B.Cu) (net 12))
 (segment (start 97.9451 81.026) (end 104.2951 87.376) (width 0.25) (layer B.Cu) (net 12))
 (segment (start 104.2951 87.376) (end 104.2951 88.7134) (width 0.25) (layer B.Cu) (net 12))
 (segment (start 104.2951 88.7134) (end 107.4701 91.8884) (width 0.25) (layer B.Cu) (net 12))
 (segment (start 107.4701 91.8884) (end 131.2584 91.8884) (width 0.25) (layer B.Cu) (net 12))
 (segment (start 131.2584 91.8884) (end 143.51 104.14) (width 0.25) (layer B.Cu) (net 12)))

